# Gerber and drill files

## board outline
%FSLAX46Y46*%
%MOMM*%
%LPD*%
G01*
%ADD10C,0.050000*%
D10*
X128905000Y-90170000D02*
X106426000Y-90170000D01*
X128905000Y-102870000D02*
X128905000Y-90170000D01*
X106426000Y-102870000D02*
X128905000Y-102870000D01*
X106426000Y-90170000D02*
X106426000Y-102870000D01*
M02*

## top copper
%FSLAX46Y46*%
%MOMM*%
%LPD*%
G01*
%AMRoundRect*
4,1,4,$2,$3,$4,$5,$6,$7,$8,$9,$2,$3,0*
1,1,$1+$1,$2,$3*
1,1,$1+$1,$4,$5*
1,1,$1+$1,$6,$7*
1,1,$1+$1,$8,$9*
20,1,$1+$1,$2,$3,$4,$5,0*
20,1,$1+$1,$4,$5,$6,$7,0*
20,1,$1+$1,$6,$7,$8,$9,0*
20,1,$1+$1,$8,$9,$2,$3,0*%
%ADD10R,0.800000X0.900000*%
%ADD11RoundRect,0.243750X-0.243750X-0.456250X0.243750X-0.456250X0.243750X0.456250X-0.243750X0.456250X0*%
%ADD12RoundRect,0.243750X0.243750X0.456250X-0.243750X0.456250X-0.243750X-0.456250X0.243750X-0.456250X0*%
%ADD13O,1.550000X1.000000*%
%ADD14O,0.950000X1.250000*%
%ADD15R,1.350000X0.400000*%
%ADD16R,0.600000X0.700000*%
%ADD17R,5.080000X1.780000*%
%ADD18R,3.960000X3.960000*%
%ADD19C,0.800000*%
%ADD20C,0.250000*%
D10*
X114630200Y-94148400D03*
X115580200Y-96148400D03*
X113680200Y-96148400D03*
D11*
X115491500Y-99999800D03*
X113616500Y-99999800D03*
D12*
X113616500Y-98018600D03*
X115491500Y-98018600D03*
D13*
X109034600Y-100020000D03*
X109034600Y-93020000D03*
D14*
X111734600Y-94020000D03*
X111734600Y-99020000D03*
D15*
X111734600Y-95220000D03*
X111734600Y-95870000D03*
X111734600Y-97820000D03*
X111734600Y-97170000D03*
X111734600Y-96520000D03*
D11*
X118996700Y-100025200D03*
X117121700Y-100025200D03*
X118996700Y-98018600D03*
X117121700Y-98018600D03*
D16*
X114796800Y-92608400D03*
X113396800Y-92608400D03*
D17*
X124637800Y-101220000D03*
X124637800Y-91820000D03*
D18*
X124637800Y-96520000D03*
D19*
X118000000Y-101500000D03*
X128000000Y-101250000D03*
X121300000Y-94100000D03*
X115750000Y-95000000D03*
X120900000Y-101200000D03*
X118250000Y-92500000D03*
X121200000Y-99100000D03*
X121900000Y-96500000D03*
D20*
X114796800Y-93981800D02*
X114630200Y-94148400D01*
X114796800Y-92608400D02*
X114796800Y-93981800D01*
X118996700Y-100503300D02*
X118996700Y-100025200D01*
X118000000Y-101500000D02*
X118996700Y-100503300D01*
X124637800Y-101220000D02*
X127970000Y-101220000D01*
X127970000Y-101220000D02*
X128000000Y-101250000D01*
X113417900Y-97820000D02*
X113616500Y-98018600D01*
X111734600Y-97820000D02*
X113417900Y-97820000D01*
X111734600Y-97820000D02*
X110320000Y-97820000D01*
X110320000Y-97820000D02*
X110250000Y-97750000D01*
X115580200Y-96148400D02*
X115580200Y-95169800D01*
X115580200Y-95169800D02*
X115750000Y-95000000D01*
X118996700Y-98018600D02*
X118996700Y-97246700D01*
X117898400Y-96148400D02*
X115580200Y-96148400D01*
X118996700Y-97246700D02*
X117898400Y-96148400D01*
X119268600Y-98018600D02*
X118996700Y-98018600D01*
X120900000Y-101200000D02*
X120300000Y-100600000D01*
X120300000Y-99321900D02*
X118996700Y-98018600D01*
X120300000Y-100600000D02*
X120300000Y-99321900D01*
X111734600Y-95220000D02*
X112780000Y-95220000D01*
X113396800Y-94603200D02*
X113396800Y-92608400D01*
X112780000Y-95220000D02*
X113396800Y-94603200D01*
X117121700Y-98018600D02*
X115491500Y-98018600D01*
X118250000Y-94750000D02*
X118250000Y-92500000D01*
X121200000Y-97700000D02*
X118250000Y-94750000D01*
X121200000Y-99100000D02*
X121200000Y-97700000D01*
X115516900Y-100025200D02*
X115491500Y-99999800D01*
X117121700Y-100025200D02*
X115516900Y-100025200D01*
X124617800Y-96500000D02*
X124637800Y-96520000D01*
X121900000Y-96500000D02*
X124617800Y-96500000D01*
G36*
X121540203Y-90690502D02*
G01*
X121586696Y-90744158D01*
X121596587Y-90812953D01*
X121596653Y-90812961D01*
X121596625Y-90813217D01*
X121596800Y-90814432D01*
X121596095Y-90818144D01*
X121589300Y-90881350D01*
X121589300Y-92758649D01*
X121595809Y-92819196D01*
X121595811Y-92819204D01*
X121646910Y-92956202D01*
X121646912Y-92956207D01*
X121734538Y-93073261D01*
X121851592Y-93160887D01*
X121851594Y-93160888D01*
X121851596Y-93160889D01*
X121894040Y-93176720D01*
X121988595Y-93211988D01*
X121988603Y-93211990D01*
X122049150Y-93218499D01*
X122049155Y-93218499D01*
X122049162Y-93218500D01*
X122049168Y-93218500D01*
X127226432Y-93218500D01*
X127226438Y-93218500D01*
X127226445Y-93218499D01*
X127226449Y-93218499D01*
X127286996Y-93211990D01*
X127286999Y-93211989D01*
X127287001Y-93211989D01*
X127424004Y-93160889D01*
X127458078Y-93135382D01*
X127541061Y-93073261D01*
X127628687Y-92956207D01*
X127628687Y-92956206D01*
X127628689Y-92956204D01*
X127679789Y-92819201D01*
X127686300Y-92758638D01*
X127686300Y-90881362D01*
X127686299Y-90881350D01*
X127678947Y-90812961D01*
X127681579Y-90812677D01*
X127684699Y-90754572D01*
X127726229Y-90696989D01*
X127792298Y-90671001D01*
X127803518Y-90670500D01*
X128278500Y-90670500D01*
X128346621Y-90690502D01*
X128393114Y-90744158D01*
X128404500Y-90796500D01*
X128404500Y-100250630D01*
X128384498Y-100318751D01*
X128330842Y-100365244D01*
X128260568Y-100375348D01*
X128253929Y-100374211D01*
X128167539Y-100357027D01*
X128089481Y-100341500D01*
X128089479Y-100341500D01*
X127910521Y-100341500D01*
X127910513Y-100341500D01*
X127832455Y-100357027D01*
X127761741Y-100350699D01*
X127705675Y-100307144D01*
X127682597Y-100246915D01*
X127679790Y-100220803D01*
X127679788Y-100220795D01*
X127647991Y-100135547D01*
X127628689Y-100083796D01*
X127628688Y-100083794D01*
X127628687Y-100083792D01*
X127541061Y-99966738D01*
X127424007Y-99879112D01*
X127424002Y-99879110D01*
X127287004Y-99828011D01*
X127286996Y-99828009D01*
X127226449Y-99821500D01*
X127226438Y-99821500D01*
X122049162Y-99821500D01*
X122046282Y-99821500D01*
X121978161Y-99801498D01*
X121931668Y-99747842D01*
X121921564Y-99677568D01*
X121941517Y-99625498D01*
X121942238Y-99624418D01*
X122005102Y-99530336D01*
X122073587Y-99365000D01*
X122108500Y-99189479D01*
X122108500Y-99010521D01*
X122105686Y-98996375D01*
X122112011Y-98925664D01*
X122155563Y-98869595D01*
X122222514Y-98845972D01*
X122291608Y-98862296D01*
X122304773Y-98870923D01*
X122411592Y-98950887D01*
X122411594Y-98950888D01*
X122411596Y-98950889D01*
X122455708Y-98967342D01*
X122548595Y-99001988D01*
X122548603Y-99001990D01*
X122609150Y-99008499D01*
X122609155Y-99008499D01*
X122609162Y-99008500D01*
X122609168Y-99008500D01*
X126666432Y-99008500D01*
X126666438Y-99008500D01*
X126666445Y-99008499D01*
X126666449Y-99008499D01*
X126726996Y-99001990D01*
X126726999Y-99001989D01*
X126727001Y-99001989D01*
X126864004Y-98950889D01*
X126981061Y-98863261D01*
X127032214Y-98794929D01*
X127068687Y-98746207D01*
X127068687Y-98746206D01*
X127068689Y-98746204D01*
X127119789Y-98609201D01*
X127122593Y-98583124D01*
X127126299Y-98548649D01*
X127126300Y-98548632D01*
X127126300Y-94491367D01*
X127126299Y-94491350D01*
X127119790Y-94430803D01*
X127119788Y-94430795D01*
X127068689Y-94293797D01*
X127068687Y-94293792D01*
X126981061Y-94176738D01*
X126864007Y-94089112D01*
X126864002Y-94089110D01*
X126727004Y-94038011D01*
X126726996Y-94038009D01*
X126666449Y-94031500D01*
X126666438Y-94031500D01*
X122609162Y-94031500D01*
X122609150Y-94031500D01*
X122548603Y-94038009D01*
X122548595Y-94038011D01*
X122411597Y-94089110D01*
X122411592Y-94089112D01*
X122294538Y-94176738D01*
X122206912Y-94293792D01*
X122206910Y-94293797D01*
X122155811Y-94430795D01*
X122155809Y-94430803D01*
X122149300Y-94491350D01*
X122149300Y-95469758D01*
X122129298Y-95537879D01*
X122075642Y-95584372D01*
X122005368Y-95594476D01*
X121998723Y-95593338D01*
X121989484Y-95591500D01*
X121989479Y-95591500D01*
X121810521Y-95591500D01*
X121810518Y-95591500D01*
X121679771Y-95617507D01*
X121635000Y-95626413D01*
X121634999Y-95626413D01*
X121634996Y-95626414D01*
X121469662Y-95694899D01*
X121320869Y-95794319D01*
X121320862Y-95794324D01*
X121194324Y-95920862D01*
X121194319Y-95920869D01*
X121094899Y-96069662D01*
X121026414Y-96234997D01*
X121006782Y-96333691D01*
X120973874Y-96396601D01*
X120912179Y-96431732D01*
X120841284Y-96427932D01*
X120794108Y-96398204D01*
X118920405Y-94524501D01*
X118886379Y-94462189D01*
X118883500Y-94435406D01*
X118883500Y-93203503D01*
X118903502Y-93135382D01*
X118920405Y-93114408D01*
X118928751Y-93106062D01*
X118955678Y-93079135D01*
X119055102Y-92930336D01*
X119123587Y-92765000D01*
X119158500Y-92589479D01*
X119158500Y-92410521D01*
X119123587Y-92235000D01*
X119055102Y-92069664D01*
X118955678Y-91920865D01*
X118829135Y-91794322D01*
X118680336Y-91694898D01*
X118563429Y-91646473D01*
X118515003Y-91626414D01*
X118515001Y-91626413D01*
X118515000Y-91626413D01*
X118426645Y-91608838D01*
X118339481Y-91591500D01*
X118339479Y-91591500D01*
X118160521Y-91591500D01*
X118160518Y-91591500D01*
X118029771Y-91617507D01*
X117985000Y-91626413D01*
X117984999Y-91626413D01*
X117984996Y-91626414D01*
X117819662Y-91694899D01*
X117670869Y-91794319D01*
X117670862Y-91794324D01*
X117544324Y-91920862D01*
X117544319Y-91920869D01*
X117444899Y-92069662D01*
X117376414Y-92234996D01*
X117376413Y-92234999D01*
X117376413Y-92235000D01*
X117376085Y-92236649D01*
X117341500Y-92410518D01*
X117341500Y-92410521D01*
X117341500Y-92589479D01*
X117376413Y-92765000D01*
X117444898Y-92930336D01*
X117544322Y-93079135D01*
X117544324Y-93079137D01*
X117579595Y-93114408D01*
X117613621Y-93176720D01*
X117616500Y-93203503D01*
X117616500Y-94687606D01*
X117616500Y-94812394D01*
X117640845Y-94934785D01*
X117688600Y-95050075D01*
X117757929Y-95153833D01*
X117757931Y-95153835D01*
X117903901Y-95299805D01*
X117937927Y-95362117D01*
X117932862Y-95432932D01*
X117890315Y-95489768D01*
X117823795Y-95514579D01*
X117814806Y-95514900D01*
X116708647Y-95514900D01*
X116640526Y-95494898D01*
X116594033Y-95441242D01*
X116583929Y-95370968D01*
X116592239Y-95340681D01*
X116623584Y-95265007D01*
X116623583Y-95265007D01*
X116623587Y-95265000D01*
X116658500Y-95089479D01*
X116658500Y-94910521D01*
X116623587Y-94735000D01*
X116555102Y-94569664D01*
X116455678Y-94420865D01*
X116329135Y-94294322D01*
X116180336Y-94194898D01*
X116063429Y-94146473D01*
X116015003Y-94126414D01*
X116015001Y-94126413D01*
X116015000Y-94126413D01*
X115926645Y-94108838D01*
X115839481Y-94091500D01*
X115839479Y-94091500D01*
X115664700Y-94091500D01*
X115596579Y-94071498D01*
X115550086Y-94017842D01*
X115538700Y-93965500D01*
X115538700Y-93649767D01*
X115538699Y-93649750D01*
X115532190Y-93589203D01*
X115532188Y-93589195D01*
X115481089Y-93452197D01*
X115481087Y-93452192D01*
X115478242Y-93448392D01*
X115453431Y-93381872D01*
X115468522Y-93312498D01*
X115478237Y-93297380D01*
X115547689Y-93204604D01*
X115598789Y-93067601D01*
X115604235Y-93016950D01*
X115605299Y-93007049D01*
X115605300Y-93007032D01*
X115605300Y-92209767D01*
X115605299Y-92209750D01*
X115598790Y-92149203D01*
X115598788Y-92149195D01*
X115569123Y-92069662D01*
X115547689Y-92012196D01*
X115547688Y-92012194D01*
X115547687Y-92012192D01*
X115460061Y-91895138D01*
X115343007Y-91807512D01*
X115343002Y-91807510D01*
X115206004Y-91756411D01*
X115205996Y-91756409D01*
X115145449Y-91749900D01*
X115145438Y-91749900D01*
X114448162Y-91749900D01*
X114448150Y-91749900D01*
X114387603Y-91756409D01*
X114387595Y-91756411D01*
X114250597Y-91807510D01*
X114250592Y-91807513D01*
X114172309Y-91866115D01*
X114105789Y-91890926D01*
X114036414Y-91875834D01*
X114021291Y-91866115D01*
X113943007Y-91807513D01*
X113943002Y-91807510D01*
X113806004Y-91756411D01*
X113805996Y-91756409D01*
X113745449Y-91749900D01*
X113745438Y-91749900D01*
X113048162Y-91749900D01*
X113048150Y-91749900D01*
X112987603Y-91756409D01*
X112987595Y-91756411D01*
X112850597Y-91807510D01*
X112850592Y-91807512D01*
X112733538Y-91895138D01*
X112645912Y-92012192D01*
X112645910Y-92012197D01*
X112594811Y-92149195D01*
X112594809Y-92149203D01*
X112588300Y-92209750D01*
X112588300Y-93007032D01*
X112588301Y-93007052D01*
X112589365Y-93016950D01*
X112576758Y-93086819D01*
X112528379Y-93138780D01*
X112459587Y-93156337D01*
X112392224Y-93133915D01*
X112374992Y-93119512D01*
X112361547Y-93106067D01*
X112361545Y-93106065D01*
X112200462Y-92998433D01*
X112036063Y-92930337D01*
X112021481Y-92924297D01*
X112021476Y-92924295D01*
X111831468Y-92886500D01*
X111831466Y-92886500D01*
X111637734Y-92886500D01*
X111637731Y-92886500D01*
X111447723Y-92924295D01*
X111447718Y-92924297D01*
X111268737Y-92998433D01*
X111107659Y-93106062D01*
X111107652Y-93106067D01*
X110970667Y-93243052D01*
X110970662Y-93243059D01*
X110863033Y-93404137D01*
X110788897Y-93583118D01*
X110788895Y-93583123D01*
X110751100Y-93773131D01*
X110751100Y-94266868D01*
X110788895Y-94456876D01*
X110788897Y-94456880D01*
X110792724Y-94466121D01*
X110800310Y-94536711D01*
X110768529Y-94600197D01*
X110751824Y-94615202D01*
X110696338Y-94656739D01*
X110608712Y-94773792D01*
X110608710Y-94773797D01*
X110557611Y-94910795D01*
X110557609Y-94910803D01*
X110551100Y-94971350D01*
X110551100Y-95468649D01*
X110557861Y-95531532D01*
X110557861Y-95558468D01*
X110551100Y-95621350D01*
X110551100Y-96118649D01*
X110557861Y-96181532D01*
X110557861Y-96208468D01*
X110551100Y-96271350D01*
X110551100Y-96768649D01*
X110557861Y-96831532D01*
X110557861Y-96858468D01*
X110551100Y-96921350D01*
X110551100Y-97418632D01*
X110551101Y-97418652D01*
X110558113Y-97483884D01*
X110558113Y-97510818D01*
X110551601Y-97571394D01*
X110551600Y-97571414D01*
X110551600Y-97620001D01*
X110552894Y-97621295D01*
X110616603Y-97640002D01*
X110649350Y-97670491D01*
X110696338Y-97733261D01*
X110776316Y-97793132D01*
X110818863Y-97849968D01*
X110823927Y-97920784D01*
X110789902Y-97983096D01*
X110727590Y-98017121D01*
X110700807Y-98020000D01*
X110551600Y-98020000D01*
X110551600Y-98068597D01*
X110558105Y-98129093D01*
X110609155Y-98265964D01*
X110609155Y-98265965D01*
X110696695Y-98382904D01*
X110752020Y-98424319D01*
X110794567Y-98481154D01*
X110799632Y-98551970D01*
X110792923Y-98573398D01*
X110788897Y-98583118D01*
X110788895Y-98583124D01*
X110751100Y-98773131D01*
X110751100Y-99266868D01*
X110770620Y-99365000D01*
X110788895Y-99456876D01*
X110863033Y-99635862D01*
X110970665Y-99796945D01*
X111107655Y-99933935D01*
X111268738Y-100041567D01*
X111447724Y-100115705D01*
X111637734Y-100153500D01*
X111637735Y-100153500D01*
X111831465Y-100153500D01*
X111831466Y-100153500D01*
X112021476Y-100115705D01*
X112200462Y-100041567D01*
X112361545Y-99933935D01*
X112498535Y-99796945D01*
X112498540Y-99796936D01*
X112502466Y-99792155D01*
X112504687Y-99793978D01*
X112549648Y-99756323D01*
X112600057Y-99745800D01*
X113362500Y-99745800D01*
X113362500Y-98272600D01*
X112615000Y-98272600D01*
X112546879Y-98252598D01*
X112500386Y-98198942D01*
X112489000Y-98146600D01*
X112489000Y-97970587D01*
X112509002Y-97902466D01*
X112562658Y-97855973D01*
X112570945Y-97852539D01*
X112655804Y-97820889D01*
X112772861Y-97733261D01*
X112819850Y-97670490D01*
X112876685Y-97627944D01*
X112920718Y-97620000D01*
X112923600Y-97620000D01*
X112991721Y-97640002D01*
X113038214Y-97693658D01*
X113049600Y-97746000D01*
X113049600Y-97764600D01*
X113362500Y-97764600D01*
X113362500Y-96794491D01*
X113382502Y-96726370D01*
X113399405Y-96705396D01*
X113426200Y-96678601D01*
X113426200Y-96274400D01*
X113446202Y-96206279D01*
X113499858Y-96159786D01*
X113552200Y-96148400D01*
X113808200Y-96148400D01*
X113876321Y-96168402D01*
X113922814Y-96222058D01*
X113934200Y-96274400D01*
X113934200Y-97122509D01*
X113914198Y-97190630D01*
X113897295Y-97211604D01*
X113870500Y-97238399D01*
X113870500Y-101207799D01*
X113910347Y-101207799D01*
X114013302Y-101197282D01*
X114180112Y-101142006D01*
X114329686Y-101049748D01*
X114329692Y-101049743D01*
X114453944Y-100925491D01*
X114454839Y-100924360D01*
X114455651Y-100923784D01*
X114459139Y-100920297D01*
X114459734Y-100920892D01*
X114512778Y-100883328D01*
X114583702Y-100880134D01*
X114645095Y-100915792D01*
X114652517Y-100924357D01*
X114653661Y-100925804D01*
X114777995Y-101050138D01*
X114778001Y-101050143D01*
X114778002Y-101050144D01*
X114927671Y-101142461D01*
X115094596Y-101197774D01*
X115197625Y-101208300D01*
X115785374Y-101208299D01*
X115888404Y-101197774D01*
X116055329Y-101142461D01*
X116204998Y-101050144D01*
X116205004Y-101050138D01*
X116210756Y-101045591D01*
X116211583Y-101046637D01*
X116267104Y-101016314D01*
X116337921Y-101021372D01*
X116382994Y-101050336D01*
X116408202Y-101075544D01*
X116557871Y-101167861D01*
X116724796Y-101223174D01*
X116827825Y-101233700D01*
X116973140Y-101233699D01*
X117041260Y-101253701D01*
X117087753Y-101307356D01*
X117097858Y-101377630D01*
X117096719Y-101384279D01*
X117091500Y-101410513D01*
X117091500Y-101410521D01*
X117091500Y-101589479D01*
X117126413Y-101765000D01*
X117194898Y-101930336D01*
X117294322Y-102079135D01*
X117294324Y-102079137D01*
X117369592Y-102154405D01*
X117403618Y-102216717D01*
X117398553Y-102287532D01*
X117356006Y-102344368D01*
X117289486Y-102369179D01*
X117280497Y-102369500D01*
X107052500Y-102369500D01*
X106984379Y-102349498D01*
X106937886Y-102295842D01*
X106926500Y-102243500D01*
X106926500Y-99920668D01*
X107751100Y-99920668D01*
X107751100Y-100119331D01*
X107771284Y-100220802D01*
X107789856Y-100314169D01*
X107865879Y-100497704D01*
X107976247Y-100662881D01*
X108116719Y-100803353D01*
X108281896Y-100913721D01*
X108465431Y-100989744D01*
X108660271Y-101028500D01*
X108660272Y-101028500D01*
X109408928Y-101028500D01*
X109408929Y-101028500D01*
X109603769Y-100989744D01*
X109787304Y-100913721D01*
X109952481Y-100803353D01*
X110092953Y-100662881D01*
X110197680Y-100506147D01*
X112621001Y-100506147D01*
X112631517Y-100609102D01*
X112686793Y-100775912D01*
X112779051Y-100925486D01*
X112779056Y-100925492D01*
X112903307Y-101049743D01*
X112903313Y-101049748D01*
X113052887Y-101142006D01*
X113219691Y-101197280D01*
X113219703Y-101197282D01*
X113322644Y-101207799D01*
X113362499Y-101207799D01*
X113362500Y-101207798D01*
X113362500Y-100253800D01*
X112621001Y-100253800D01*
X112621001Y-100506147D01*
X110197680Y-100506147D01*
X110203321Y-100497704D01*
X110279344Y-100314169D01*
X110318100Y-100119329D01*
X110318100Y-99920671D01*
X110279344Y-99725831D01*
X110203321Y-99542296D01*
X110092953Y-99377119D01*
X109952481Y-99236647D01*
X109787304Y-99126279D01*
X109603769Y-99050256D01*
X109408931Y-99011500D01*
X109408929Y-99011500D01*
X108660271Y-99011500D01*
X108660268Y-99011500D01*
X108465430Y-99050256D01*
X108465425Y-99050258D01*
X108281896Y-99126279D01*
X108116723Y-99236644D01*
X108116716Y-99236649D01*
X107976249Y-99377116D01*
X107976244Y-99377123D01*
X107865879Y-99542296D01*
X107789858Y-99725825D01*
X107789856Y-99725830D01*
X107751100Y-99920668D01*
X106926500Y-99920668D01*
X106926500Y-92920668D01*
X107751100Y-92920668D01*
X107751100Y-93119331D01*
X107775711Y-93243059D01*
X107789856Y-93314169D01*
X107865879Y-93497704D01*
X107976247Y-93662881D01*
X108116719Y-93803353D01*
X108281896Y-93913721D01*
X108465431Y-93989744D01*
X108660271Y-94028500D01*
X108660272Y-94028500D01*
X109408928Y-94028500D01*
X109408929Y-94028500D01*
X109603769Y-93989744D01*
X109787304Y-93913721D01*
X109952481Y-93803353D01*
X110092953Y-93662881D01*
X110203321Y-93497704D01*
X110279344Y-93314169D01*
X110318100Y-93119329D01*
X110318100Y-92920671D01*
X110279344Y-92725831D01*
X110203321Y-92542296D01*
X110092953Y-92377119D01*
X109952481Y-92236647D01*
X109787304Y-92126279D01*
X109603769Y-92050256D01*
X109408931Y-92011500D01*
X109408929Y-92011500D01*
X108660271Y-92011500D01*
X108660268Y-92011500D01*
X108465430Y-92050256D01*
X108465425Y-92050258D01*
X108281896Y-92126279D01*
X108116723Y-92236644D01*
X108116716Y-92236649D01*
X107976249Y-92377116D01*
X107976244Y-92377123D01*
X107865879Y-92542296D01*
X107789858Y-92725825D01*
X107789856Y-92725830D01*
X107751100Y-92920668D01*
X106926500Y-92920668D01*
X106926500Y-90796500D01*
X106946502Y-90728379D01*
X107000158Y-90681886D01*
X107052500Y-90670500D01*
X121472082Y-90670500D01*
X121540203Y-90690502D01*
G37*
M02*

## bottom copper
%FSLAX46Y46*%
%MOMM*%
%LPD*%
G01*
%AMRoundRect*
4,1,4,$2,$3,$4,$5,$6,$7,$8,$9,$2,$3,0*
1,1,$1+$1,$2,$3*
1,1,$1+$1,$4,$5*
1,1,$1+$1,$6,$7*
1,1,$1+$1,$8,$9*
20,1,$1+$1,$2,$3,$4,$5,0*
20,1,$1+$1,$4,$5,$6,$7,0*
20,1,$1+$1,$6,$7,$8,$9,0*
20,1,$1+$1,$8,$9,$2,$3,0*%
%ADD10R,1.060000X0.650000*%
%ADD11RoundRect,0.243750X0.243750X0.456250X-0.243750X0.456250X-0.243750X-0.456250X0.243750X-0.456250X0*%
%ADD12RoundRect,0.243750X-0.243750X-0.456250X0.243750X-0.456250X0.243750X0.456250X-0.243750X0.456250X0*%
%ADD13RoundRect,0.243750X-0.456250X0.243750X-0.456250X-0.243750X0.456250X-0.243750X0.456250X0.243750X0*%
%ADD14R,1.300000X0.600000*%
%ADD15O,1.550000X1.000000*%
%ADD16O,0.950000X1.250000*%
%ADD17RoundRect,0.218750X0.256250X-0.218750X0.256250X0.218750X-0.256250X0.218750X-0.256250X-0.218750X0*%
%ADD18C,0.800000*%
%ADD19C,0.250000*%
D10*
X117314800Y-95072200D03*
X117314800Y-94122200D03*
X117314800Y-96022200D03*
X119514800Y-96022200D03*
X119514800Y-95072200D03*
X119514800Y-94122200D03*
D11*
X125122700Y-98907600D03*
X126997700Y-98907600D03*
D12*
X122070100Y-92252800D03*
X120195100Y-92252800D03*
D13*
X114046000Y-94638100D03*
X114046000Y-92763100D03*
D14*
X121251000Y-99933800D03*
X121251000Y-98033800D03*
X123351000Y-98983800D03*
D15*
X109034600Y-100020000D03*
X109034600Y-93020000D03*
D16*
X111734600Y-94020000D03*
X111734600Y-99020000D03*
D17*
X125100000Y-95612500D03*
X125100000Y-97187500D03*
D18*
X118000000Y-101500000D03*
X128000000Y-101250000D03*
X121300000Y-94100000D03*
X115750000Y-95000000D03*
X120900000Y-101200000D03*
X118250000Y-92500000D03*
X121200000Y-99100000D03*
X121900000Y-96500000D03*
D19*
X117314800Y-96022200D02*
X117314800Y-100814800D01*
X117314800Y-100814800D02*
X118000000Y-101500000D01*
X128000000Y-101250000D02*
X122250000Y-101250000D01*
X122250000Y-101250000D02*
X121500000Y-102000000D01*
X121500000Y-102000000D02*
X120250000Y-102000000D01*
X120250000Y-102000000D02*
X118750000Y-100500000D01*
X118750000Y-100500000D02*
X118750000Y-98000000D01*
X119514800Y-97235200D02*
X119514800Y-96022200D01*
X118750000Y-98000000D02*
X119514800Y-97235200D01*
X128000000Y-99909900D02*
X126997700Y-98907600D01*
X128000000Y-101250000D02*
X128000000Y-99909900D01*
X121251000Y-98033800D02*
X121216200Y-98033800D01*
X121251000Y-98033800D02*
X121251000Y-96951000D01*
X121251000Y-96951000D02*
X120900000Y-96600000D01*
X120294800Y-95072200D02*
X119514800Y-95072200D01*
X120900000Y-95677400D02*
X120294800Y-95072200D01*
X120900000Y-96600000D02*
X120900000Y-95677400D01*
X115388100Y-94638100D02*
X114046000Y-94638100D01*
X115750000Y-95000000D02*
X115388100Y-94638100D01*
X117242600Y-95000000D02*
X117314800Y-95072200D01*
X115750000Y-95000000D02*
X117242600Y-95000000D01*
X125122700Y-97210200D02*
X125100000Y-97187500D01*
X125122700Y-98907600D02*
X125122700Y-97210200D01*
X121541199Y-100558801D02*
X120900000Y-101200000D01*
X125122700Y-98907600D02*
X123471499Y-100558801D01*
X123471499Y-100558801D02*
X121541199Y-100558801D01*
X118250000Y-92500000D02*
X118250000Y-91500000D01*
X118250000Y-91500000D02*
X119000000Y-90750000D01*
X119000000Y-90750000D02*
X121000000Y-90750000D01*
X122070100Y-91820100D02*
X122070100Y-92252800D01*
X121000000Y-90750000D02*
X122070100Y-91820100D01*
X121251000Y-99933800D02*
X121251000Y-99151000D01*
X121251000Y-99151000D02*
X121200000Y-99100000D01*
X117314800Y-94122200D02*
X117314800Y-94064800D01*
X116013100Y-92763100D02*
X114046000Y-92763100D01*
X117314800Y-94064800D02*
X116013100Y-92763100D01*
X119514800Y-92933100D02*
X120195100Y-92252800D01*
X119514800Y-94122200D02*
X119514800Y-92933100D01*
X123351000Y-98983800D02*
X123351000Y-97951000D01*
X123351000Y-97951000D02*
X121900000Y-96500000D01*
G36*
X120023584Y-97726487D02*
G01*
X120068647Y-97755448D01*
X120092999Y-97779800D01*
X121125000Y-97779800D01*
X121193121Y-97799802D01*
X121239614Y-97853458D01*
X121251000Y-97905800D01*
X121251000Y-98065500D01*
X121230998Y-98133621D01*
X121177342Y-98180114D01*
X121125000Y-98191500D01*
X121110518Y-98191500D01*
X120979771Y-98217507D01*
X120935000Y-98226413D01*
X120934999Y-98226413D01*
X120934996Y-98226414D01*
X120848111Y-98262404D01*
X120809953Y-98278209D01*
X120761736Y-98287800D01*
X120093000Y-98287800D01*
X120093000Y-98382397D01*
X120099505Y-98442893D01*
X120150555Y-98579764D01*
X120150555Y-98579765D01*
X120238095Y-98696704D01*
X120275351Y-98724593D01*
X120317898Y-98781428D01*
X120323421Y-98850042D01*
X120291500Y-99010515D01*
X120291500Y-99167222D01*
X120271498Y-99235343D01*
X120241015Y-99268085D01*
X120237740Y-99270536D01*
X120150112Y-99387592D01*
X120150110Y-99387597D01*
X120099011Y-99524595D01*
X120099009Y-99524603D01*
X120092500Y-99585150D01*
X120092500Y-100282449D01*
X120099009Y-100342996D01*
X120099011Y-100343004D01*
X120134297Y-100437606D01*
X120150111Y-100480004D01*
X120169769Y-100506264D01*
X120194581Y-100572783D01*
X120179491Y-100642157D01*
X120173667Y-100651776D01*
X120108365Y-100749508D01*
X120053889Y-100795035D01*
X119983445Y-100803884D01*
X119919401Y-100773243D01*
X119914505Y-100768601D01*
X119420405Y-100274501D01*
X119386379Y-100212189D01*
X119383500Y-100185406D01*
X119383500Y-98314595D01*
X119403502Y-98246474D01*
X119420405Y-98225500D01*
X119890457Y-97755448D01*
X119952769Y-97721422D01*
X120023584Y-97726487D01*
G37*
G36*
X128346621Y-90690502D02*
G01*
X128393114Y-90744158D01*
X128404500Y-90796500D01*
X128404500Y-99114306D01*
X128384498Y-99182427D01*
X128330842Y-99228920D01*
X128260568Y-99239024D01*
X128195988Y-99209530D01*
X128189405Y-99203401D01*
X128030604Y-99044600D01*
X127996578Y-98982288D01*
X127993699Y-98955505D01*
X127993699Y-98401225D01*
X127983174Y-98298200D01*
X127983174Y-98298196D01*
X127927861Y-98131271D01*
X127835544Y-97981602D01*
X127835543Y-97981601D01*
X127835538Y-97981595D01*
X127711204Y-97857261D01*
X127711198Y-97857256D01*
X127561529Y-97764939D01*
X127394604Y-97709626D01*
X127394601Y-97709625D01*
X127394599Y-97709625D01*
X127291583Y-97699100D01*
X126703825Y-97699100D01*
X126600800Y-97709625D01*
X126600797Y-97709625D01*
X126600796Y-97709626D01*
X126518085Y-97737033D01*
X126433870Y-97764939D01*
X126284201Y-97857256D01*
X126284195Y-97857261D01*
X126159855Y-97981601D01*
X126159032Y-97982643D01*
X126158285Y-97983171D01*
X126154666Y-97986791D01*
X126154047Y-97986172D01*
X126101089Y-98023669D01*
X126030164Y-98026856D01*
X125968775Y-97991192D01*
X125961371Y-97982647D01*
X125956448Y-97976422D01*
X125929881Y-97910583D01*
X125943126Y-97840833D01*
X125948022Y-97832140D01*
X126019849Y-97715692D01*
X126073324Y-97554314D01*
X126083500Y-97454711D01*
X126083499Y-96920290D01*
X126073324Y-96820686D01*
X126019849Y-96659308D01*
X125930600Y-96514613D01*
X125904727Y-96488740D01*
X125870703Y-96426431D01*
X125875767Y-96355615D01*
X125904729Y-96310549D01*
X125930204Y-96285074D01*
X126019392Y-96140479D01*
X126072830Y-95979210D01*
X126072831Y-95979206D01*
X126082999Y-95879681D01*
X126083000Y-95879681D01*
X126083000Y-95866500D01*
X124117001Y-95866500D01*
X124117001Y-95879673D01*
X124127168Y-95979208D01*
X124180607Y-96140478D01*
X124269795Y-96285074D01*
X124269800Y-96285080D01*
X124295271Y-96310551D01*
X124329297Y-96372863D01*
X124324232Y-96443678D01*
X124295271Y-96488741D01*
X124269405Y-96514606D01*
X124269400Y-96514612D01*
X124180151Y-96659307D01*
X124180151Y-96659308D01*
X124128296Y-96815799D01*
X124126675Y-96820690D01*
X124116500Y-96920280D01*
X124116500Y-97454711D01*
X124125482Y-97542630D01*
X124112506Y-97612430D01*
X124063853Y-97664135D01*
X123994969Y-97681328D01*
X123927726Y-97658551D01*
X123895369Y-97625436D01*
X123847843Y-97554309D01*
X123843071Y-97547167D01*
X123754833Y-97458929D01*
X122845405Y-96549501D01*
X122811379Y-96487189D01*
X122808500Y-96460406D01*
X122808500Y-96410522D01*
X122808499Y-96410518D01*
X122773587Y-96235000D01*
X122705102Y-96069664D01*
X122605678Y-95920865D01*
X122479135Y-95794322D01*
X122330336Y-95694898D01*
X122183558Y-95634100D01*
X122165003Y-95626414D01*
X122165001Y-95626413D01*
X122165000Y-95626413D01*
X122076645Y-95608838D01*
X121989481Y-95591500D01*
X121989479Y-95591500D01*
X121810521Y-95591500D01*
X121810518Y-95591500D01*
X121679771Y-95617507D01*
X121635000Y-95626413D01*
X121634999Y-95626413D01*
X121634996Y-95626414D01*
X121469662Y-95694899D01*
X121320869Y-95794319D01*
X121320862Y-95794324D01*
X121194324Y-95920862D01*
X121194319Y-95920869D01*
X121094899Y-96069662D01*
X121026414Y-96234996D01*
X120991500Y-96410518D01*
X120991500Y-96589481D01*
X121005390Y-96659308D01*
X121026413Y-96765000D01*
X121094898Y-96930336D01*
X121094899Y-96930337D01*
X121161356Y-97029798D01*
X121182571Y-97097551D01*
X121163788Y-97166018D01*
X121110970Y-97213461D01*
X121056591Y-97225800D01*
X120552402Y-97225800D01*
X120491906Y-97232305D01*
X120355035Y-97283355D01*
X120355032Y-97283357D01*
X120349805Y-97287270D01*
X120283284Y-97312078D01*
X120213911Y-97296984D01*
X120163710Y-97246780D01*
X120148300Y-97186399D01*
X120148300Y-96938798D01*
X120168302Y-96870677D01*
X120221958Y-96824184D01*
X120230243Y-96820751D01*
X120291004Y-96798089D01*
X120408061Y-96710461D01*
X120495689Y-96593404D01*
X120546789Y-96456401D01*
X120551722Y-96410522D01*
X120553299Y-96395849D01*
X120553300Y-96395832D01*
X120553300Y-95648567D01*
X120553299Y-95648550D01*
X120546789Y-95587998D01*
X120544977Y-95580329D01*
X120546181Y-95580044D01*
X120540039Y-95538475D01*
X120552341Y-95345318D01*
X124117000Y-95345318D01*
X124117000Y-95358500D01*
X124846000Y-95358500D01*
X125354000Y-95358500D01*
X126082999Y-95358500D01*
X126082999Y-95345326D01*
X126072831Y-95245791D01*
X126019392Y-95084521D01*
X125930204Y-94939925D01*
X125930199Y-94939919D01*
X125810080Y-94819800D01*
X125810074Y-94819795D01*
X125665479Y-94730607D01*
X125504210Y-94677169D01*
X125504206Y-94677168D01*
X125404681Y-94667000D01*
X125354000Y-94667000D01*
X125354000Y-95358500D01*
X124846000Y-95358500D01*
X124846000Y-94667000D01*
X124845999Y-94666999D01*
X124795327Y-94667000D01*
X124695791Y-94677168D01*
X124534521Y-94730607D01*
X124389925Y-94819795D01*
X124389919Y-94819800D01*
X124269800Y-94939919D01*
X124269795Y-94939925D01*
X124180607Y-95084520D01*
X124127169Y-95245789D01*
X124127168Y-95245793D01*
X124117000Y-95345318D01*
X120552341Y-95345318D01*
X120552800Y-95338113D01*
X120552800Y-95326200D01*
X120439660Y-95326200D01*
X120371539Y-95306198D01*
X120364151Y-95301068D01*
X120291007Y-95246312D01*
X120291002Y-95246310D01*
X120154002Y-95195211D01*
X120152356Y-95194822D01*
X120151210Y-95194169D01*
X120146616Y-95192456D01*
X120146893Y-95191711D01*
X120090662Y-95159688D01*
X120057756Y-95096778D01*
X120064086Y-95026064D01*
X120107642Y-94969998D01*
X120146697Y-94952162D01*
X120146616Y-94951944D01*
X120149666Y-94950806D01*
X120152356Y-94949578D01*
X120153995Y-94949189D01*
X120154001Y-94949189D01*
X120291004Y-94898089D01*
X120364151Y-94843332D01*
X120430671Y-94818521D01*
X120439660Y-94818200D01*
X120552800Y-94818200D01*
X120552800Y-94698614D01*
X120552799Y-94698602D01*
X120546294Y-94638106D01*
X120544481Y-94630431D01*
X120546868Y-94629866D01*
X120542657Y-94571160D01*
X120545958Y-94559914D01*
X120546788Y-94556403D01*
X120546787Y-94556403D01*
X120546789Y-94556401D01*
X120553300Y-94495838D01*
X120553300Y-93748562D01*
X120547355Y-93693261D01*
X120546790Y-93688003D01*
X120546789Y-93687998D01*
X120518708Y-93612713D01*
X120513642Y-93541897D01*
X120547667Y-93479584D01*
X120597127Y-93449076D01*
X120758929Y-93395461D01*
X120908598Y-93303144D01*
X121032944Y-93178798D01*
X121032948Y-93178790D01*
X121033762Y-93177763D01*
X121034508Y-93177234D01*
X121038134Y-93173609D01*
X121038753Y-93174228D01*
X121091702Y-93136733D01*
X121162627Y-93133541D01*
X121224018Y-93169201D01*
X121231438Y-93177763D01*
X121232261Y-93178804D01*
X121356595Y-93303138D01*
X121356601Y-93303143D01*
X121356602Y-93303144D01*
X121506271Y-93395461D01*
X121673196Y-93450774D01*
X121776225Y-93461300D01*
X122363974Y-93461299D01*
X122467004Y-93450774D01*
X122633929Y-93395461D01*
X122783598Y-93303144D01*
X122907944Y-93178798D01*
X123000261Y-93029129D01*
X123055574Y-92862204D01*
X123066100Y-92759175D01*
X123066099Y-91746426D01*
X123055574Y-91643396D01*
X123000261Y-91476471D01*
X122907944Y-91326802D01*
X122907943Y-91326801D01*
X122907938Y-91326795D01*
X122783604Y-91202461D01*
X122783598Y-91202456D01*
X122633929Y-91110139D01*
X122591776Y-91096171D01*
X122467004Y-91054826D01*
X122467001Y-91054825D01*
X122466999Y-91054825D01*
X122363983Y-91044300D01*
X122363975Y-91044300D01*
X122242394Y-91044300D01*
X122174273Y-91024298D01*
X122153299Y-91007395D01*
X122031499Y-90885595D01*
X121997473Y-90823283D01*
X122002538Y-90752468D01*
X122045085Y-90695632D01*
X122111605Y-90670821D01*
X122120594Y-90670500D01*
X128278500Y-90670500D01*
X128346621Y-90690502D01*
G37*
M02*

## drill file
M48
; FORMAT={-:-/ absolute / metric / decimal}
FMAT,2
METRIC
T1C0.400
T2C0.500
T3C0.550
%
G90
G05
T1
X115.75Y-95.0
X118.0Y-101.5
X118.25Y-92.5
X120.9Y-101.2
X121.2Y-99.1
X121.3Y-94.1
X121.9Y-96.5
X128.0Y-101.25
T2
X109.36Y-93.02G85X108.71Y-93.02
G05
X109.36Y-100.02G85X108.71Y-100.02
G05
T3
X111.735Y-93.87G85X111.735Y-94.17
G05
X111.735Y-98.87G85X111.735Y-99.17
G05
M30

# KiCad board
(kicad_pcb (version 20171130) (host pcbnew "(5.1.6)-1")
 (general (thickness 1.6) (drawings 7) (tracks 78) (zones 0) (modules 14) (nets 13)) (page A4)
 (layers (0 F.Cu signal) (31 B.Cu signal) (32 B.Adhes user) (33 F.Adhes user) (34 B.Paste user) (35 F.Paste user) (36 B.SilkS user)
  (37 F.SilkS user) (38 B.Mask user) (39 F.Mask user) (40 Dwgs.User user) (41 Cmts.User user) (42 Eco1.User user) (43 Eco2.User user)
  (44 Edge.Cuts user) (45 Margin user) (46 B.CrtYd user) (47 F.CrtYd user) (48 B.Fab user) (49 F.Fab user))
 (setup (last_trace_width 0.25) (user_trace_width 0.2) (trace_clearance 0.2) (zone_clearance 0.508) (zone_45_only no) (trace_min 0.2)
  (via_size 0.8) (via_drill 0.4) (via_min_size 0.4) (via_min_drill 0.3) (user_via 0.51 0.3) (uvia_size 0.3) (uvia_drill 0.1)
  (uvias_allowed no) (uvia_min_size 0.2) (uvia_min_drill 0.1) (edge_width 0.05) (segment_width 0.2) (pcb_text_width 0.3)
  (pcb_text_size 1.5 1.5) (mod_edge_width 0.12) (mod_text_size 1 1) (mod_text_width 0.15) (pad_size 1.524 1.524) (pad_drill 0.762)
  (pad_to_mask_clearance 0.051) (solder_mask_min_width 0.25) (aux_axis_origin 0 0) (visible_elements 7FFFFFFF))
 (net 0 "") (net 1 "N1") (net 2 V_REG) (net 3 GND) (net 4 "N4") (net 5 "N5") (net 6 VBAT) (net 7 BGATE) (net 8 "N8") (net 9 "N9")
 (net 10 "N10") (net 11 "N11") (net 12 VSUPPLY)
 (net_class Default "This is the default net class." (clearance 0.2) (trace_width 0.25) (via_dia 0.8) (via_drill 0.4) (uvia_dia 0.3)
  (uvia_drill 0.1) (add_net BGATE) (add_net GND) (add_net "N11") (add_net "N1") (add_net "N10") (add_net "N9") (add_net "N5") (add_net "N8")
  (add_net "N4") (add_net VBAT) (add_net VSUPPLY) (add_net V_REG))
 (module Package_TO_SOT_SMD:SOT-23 (layer F.Cu) (at 114.6302 95.1484 90)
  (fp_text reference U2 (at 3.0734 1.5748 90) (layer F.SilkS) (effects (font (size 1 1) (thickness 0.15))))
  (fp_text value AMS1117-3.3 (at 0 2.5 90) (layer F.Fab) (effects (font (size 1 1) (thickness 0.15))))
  (pad 3 smd rect (at 1 0 90) (size 0.9 0.8) (layers F.Cu F.Paste F.Mask) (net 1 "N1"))
  (pad 2 smd rect (at -1 0.95 90) (size 0.9 0.8) (layers F.Cu F.Paste F.Mask) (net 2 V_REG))
  (pad 1 smd rect (at -1 -0.95 90) (size 0.9 0.8) (layers F.Cu F.Paste F.Mask) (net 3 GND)))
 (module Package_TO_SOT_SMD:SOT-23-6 (layer B.Cu) (at 118.4148 95.0722 180)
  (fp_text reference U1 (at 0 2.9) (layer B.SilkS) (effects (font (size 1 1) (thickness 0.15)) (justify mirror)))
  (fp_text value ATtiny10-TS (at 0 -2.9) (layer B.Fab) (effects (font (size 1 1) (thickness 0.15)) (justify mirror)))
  (pad 5 smd rect (at 1.1 0 180) (size 1.06 0.65) (layers B.Cu B.Paste B.Mask) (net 2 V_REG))
  (pad 6 smd rect (at 1.1 0.95 180) (size 1.06 0.65) (layers B.Cu B.Paste B.Mask) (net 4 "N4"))
  (pad 4 smd rect (at 1.1 -0.95 180) (size 1.06 0.65) (layers B.Cu B.Paste B.Mask) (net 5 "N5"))
  (pad 3 smd rect (at -1.1 -0.95 180) (size 1.06 0.65) (layers B.Cu B.Paste B.Mask) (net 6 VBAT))
  (pad 2 smd rect (at -1.1 0 180) (size 1.06 0.65) (layers B.Cu B.Paste B.Mask) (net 3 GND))
  (pad 1 smd rect (at -1.1 0.95 180) (size 1.06 0.65) (layers B.Cu B.Paste B.Mask) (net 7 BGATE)))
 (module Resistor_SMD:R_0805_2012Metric (layer B.Cu) (at 126.0602 98.9076 180)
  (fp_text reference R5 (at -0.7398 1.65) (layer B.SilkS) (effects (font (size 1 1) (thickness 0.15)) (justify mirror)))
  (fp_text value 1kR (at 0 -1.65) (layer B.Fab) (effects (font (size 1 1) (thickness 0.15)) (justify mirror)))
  (pad 2 smd roundrect (at 0.9375 0 180) (size 0.975 1.4) (layers B.Cu B.Paste B.Mask) (roundrect_rratio 0.25) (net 2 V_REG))
  (pad 1 smd roundrect (at -0.9375 0 180) (size 0.975 1.4) (layers B.Cu B.Paste B.Mask) (roundrect_rratio 0.25) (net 6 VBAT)))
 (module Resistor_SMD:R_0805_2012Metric (layer B.Cu) (at 121.1326 92.2528)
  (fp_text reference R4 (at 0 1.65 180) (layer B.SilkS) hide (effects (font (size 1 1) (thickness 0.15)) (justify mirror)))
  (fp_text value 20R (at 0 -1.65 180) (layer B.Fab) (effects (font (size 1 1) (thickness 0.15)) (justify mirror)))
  (pad 2 smd roundrect (at 0.9375 0) (size 0.975 1.4) (layers B.Cu B.Paste B.Mask) (roundrect_rratio 0.25) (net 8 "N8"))
  (pad 1 smd roundrect (at -0.9375 0) (size 0.975 1.4) (layers B.Cu B.Paste B.Mask) (roundrect_rratio 0.25) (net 7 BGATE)))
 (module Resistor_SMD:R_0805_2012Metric (layer F.Cu) (at 114.554 99.9998)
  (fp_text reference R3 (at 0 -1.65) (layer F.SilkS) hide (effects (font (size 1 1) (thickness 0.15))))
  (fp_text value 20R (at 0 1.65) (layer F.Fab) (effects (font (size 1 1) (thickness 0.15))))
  (pad 2 smd roundrect (at 0.9375 0) (size 0.975 1.4) (layers F.Cu F.Paste F.Mask) (roundrect_rratio 0.25) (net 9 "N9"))
  (pad 1 smd roundrect (at -0.9375 0) (size 0.975 1.4) (layers F.Cu F.Paste F.Mask) (roundrect_rratio 0.25) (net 3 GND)))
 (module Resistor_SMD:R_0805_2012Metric (layer B.Cu) (at 114.046 93.7006 270)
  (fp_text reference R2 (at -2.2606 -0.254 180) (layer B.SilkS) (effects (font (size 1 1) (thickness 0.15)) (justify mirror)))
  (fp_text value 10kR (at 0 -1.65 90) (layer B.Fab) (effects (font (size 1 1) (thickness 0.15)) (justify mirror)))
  (pad 2 smd roundrect (at 0.9375 0 270) (size 0.975 1.4) (layers B.Cu B.Paste B.Mask) (roundrect_rratio 0.25) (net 2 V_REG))
  (pad 1 smd roundrect (at -0.9375 0 270) (size 0.975 1.4) (layers B.Cu B.Paste B.Mask) (roundrect_rratio 0.25) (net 4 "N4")))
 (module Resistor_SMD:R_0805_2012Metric (layer F.Cu) (at 114.554 98.0186 180)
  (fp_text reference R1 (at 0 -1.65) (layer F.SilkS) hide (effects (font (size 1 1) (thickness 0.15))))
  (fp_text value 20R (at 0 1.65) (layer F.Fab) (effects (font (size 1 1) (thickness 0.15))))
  (pad 2 smd roundrect (at 0.9375 0 180) (size 0.975 1.4) (layers F.Cu F.Paste F.Mask) (roundrect_rratio 0.25) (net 3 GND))
  (pad 1 smd roundrect (at -0.9375 0 180) (size 0.975 1.4) (layers F.Cu F.Paste F.Mask) (roundrect_rratio 0.25) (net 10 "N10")))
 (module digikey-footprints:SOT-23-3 (layer B.Cu) (at 122.301 98.9838)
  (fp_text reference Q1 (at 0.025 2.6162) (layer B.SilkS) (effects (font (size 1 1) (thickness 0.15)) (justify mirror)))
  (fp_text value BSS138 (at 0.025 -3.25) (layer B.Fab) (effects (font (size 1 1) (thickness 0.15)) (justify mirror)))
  (pad 1 smd rect (at -1.05 0.95) (size 1.3 0.6) (layers B.Cu B.Paste B.Mask) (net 8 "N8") (solder_mask_margin 0.07))
  (pad 2 smd rect (at -1.05 -0.95) (size 1.3 0.6) (layers B.Cu B.Paste B.Mask) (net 3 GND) (solder_mask_margin 0.07))
  (pad 3 smd rect (at 1.05 0) (size 1.3 0.6) (layers B.Cu B.Paste B.Mask) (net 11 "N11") (solder_mask_margin 0.07)))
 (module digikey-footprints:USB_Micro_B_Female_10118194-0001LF (layer F.Cu) (at 111.7346 96.52 270)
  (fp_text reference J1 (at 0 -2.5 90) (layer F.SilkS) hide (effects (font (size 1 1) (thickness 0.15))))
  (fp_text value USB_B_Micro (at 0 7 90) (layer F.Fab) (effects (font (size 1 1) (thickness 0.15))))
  (pad SH thru_hole oval (at 3.5 2.7 270) (size 1 1.55) (drill oval 0.5 1.15) (layers *.Cu *.Mask))
  (pad SH thru_hole oval (at -3.5 2.7 270) (size 1 1.55) (drill oval 0.5 1.15) (layers *.Cu *.Mask))
  (pad SH thru_hole oval (at -2.5 0 270) (size 1.25 0.95) (drill oval 0.85 0.55) (layers *.Cu *.Mask))
  (pad SH thru_hole oval (at 2.5 0 270) (size 1.25 0.95) (drill oval 0.85 0.55) (layers *.Cu *.Mask))
  (pad 1 smd rect (at -1.3 0 270) (size 0.4 1.35) (layers F.Cu F.Paste F.Mask) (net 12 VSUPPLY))
  (pad 2 smd rect (at -0.65 0 270) (size 0.4 1.35) (layers F.Cu F.Paste F.Mask))
  (pad 5 smd rect (at 1.3 0 270) (size 0.4 1.35) (layers F.Cu F.Paste F.Mask) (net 3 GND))
  (pad 4 smd rect (at 0.65 0 270) (size 0.4 1.35) (layers F.Cu F.Paste F.Mask))
  (pad 3 smd rect (at 0 0 270) (size 0.4 1.35) (layers F.Cu F.Paste F.Mask)))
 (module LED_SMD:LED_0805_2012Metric (layer F.Cu) (at 118.0592 100.0252)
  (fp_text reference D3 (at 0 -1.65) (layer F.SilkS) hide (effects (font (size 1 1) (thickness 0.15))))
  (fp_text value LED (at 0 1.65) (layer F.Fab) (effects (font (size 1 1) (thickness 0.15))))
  (pad 2 smd roundrect (at 0.9375 0) (size 0.975 1.4) (layers F.Cu F.Paste F.Mask) (roundrect_rratio 0.25) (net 5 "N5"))
  (pad 1 smd roundrect (at -0.9375 0) (size 0.975 1.4) (layers F.Cu F.Paste F.Mask) (roundrect_rratio 0.25) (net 9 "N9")))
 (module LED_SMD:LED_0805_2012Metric (layer F.Cu) (at 118.0592 98.0186)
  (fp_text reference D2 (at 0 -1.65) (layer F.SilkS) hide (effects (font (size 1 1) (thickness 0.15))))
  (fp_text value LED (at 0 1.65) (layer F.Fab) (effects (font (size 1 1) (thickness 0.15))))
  (pad 2 smd roundrect (at 0.9375 0) (size 0.975 1.4) (layers F.Cu F.Paste F.Mask) (roundrect_rratio 0.25) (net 2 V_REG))
  (pad 1 smd roundrect (at -0.9375 0) (size 0.975 1.4) (layers F.Cu F.Paste F.Mask) (roundrect_rratio 0.25) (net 10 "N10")))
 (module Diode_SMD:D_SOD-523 (layer F.Cu) (at 114.0968 92.6084 180)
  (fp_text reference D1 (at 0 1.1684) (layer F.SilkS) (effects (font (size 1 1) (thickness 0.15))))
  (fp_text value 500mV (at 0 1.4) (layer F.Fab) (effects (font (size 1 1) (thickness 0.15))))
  (pad 1 smd rect (at -0.7 0) (size 0.6 0.7) (layers F.Cu F.Paste F.Mask) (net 1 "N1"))
  (pad 2 smd rect (at 0.7 0) (size 0.6 0.7) (layers F.Cu F.Paste F.Mask) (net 12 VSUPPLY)))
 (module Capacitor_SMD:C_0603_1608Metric (layer B.Cu) (at 125.1 96.4 90)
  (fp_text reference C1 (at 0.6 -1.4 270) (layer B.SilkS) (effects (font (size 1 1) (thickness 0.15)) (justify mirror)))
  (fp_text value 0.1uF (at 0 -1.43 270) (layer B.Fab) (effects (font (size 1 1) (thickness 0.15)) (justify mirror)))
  (pad 2 smd roundrect (at 0.7875 0 90) (size 0.875 0.95) (layers B.Cu B.Paste B.Mask) (roundrect_rratio 0.25) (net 3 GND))
  (pad 1 smd roundrect (at -0.7875 0 90) (size 0.875 0.95) (layers B.Cu B.Paste B.Mask) (roundrect_rratio 0.25) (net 2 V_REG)))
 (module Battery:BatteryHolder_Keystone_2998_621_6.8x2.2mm (layer F.Cu) (at 124.6378 96.52 270)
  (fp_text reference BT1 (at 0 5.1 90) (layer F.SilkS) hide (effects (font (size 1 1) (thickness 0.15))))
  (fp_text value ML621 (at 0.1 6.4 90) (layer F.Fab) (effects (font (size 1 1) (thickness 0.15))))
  (pad 1 smd rect (at 4.7 0 270) (size 1.78 5.08) (layers F.Cu F.Paste F.Mask) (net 6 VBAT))
  (pad 3 smd rect (at -4.7 0 270) (size 1.78 5.08) (layers F.Cu F.Paste F.Mask))
  (pad 2 smd rect (at 0 0 270) (size 3.96 3.96) (layers F.Cu F.Paste F.Mask) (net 11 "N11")))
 (gr_line (start 128.905 90.17) (end 106.426 90.17) (layer Edge.Cuts) (width 0.05))
 (gr_line (start 128.905 102.87) (end 128.905 90.17) (layer Edge.Cuts) (width 0.05))
 (gr_line (start 106.426 102.87) (end 128.905 102.87) (layer Edge.Cuts) (width 0.05))
 (gr_line (start 106.426 90.17) (end 106.426 102.87) (layer Edge.Cuts) (width 0.05))
 (segment (start 114.7968 93.9818) (end 114.6302 94.1484) (width 0.25) (layer F.Cu) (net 1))
 (segment (start 114.7968 92.6084) (end 114.7968 93.9818) (width 0.25) (layer F.Cu) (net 1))
 (via (at 118 101.5) (size 0.8) (drill 0.4) (layers F.Cu B.Cu) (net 5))
 (segment (start 117.3148 96.0222) (end 117.3148 100.8148) (width 0.25) (layer B.Cu) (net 5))
 (segment (start 117.3148 100.8148) (end 118 101.5) (width 0.25) (layer B.Cu) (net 5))
 (segment (start 118.9967 100.5033) (end 118.9967 100.0252) (width 0.25) (layer F.Cu) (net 5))
 (segment (start 118 101.5) (end 118.9967 100.5033) (width 0.25) (layer F.Cu) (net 5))
 (via (at 128 101.25) (size 0.8) (drill 0.4) (layers F.Cu B.Cu) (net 6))
 (segment (start 124.6378 101.22) (end 127.97 101.22) (width 0.25) (layer F.Cu) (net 6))
 (segment (start 127.97 101.22) (end 128 101.25) (width 0.25) (layer F.Cu) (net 6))
 (segment (start 128 101.25) (end 122.25 101.25) (width 0.25) (layer B.Cu) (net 6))
 (segment (start 122.25 101.25) (end 121.5 102) (width 0.25) (layer B.Cu) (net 6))
 (segment (start 121.5 102) (end 120.25 102) (width 0.25) (layer B.Cu) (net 6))
 (segment (start 120.25 102) (end 118.75 100.5) (width 0.25) (layer B.Cu) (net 6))
 (segment (start 118.75 100.5) (end 118.75 98) (width 0.25) (layer B.Cu) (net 6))
 (segment (start 119.5148 97.2352) (end 119.5148 96.0222) (width 0.25) (layer B.Cu) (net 6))
 (segment (start 118.75 98) (end 119.5148 97.2352) (width 0.25) (layer B.Cu) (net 6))
 (segment (start 128 99.9099) (end 126.9977 98.9076) (width 0.25) (layer B.Cu) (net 6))
 (segment (start 128 101.25) (end 128 99.9099) (width 0.25) (layer B.Cu) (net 6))
 (segment (start 113.4179 97.82) (end 113.6165 98.0186) (width 0.25) (layer F.Cu) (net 3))
 (segment (start 111.7346 97.82) (end 113.4179 97.82) (width 0.25) (layer F.Cu) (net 3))
 (segment (start 111.7346 97.82) (end 110.32 97.82) (width 0.25) (layer F.Cu) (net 3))
 (segment (start 110.32 97.82) (end 110.25 97.75) (width 0.25) (layer F.Cu) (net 3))
 (segment (start 121.251 98.0338) (end 121.2162 98.0338) (width 0.25) (layer B.Cu) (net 3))
 (segment (start 121.251 98.0338) (end 121.251 96.951) (width 0.25) (layer B.Cu) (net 3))
 (segment (start 121.251 96.951) (end 120.9 96.6) (width 0.25) (layer B.Cu) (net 3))
 (segment (start 120.2948 95.0722) (end 119.5148 95.0722) (width 0.25) (layer B.Cu) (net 3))
 (segment (start 120.9 95.6774) (end 120.2948 95.0722) (width 0.25) (layer B.Cu) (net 3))
 (segment (start 120.9 96.6) (end 120.9 95.6774) (width 0.25) (layer B.Cu) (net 3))
 (via (at 121.3 94.1) (size 0.8) (drill 0.4) (layers F.Cu B.Cu) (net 3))
 (via (at 115.75 95) (size 0.8) (drill 0.4) (layers F.Cu B.Cu) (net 2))
 (segment (start 115.5802 96.1484) (end 115.5802 95.1698) (width 0.25) (layer F.Cu) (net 2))
 (segment (start 115.5802 95.1698) (end 115.75 95) (width 0.25) (layer F.Cu) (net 2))
 (segment (start 115.3881 94.6381) (end 114.046 94.6381) (width 0.25) (layer B.Cu) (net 2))
 (segment (start 115.75 95) (end 115.3881 94.6381) (width 0.25) (layer B.Cu) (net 2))
 (segment (start 117.2426 95) (end 117.3148 95.0722) (width 0.25) (layer B.Cu) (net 2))
 (segment (start 115.75 95) (end 117.2426 95) (width 0.25) (layer B.Cu) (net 2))
 (segment (start 118.9967 98.0186) (end 118.9967 97.2467) (width 0.25) (layer F.Cu) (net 2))
 (segment (start 117.8984 96.1484) (end 115.5802 96.1484) (width 0.25) (layer F.Cu) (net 2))
 (segment (start 118.9967 97.2467) (end 117.8984 96.1484) (width 0.25) (layer F.Cu) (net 2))
 (segment (start 119.2686 98.0186) (end 118.9967 98.0186) (width 0.25) (layer F.Cu) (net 2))
 (segment (start 125.1227 97.2102) (end 125.1 97.1875) (width 0.25) (layer B.Cu) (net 2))
 (segment (start 125.1227 98.9076) (end 125.1227 97.2102) (width 0.25) (layer B.Cu) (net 2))
 (via (at 120.9 101.2) (size 0.8) (drill 0.4) (layers F.Cu B.Cu) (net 2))
 (segment (start 121.541199 100.558801) (end 120.9 101.2) (width 0.25) (layer B.Cu) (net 2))
 (segment (start 125.1227 98.9076) (end 123.471499 100.558801) (width 0.25) (layer B.Cu) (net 2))
 (segment (start 123.471499 100.558801) (end 121.541199 100.558801) (width 0.25) (layer B.Cu) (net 2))
 (segment (start 120.9 101.2) (end 120.3 100.6) (width 0.25) (layer F.Cu) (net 2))
 (segment (start 120.3 99.3219) (end 118.9967 98.0186) (width 0.25) (layer F.Cu) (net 2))
 (segment (start 120.3 100.6) (end 120.3 99.3219) (width 0.25) (layer F.Cu) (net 2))
 (segment (start 111.7346 95.22) (end 112.78 95.22) (width 0.25) (layer F.Cu) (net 12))
 (segment (start 113.3968 94.6032) (end 113.3968 92.6084) (width 0.25) (layer F.Cu) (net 12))
 (segment (start 112.78 95.22) (end 113.3968 94.6032) (width 0.25) (layer F.Cu) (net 12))
 (segment (start 117.1217 98.0186) (end 115.4915 98.0186) (width 0.25) (layer F.Cu) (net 10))
 (via (at 118.25 92.5) (size 0.8) (drill 0.4) (layers F.Cu B.Cu) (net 8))
 (segment (start 118.25 94.75) (end 118.25 92.5) (width 0.25) (layer F.Cu) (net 8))
 (segment (start 118.25 92.5) (end 118.25 91.5) (width 0.25) (layer B.Cu) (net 8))
 (segment (start 118.25 91.5) (end 119 90.75) (width 0.25) (layer B.Cu) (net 8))
 (segment (start 119 90.75) (end 121 90.75) (width 0.25) (layer B.Cu) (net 8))
 (segment (start 122.0701 91.8201) (end 122.0701 92.2528) (width 0.25) (layer B.Cu) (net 8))
 (segment (start 121 90.75) (end 122.0701 91.8201) (width 0.25) (layer B.Cu) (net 8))
 (via (at 121.2 99.1) (size 0.8) (drill 0.4) (layers F.Cu B.Cu) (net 8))
 (segment (start 121.251 99.9338) (end 121.251 99.151) (width 0.25) (layer B.Cu) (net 8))
 (segment (start 121.251 99.151) (end 121.2 99.1) (width 0.25) (layer B.Cu) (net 8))
 (segment (start 121.2 97.7) (end 118.25 94.75) (width 0.25) (layer F.Cu) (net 8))
 (segment (start 121.2 99.1) (end 121.2 97.7) (width 0.25) (layer F.Cu) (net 8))
 (segment (start 117.3148 94.1222) (end 117.3148 94.0648) (width 0.25) (layer B.Cu) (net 4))
 (segment (start 116.0131 92.7631) (end 114.046 92.7631) (width 0.25) (layer B.Cu) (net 4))
 (segment (start 117.3148 94.0648) (end 116.0131 92.7631) (width 0.25) (layer B.Cu) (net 4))
 (segment (start 119.5148 92.9331) (end 120.1951 92.2528) (width 0.25) (layer B.Cu) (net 7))
 (segment (start 119.5148 94.1222) (end 119.5148 92.9331) (width 0.25) (layer B.Cu) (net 7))
 (segment (start 115.5169 100.0252) (end 115.4915 99.9998) (width 0.25) (layer F.Cu) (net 9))
 (segment (start 117.1217 100.0252) (end 115.5169 100.0252) (width 0.25) (layer F.Cu) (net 9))
 (via (at 121.9 96.5) (size 0.8) (drill 0.4) (layers F.Cu B.Cu) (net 11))
 (segment (start 123.351 98.9838) (end 123.351 97.951) (width 0.25) (layer B.Cu) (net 11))
 (segment (start 123.351 97.951) (end 121.9 96.5) (width 0.25) (layer B.Cu) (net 11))
 (segment (start 124.6178 96.5) (end 124.6378 96.52) (width 0.25) (layer F.Cu) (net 11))
 (segment (start 121.9 96.5) (end 124.6178 96.5) (width 0.25) (layer F.Cu) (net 11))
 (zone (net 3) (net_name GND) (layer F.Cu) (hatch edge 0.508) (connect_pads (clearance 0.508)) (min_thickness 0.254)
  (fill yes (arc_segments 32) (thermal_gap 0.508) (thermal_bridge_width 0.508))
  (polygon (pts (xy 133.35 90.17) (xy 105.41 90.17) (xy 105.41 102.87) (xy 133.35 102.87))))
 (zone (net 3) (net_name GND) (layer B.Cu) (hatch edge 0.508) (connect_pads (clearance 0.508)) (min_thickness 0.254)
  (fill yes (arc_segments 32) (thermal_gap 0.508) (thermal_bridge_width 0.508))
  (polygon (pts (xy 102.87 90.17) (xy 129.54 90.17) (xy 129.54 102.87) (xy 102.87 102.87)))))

